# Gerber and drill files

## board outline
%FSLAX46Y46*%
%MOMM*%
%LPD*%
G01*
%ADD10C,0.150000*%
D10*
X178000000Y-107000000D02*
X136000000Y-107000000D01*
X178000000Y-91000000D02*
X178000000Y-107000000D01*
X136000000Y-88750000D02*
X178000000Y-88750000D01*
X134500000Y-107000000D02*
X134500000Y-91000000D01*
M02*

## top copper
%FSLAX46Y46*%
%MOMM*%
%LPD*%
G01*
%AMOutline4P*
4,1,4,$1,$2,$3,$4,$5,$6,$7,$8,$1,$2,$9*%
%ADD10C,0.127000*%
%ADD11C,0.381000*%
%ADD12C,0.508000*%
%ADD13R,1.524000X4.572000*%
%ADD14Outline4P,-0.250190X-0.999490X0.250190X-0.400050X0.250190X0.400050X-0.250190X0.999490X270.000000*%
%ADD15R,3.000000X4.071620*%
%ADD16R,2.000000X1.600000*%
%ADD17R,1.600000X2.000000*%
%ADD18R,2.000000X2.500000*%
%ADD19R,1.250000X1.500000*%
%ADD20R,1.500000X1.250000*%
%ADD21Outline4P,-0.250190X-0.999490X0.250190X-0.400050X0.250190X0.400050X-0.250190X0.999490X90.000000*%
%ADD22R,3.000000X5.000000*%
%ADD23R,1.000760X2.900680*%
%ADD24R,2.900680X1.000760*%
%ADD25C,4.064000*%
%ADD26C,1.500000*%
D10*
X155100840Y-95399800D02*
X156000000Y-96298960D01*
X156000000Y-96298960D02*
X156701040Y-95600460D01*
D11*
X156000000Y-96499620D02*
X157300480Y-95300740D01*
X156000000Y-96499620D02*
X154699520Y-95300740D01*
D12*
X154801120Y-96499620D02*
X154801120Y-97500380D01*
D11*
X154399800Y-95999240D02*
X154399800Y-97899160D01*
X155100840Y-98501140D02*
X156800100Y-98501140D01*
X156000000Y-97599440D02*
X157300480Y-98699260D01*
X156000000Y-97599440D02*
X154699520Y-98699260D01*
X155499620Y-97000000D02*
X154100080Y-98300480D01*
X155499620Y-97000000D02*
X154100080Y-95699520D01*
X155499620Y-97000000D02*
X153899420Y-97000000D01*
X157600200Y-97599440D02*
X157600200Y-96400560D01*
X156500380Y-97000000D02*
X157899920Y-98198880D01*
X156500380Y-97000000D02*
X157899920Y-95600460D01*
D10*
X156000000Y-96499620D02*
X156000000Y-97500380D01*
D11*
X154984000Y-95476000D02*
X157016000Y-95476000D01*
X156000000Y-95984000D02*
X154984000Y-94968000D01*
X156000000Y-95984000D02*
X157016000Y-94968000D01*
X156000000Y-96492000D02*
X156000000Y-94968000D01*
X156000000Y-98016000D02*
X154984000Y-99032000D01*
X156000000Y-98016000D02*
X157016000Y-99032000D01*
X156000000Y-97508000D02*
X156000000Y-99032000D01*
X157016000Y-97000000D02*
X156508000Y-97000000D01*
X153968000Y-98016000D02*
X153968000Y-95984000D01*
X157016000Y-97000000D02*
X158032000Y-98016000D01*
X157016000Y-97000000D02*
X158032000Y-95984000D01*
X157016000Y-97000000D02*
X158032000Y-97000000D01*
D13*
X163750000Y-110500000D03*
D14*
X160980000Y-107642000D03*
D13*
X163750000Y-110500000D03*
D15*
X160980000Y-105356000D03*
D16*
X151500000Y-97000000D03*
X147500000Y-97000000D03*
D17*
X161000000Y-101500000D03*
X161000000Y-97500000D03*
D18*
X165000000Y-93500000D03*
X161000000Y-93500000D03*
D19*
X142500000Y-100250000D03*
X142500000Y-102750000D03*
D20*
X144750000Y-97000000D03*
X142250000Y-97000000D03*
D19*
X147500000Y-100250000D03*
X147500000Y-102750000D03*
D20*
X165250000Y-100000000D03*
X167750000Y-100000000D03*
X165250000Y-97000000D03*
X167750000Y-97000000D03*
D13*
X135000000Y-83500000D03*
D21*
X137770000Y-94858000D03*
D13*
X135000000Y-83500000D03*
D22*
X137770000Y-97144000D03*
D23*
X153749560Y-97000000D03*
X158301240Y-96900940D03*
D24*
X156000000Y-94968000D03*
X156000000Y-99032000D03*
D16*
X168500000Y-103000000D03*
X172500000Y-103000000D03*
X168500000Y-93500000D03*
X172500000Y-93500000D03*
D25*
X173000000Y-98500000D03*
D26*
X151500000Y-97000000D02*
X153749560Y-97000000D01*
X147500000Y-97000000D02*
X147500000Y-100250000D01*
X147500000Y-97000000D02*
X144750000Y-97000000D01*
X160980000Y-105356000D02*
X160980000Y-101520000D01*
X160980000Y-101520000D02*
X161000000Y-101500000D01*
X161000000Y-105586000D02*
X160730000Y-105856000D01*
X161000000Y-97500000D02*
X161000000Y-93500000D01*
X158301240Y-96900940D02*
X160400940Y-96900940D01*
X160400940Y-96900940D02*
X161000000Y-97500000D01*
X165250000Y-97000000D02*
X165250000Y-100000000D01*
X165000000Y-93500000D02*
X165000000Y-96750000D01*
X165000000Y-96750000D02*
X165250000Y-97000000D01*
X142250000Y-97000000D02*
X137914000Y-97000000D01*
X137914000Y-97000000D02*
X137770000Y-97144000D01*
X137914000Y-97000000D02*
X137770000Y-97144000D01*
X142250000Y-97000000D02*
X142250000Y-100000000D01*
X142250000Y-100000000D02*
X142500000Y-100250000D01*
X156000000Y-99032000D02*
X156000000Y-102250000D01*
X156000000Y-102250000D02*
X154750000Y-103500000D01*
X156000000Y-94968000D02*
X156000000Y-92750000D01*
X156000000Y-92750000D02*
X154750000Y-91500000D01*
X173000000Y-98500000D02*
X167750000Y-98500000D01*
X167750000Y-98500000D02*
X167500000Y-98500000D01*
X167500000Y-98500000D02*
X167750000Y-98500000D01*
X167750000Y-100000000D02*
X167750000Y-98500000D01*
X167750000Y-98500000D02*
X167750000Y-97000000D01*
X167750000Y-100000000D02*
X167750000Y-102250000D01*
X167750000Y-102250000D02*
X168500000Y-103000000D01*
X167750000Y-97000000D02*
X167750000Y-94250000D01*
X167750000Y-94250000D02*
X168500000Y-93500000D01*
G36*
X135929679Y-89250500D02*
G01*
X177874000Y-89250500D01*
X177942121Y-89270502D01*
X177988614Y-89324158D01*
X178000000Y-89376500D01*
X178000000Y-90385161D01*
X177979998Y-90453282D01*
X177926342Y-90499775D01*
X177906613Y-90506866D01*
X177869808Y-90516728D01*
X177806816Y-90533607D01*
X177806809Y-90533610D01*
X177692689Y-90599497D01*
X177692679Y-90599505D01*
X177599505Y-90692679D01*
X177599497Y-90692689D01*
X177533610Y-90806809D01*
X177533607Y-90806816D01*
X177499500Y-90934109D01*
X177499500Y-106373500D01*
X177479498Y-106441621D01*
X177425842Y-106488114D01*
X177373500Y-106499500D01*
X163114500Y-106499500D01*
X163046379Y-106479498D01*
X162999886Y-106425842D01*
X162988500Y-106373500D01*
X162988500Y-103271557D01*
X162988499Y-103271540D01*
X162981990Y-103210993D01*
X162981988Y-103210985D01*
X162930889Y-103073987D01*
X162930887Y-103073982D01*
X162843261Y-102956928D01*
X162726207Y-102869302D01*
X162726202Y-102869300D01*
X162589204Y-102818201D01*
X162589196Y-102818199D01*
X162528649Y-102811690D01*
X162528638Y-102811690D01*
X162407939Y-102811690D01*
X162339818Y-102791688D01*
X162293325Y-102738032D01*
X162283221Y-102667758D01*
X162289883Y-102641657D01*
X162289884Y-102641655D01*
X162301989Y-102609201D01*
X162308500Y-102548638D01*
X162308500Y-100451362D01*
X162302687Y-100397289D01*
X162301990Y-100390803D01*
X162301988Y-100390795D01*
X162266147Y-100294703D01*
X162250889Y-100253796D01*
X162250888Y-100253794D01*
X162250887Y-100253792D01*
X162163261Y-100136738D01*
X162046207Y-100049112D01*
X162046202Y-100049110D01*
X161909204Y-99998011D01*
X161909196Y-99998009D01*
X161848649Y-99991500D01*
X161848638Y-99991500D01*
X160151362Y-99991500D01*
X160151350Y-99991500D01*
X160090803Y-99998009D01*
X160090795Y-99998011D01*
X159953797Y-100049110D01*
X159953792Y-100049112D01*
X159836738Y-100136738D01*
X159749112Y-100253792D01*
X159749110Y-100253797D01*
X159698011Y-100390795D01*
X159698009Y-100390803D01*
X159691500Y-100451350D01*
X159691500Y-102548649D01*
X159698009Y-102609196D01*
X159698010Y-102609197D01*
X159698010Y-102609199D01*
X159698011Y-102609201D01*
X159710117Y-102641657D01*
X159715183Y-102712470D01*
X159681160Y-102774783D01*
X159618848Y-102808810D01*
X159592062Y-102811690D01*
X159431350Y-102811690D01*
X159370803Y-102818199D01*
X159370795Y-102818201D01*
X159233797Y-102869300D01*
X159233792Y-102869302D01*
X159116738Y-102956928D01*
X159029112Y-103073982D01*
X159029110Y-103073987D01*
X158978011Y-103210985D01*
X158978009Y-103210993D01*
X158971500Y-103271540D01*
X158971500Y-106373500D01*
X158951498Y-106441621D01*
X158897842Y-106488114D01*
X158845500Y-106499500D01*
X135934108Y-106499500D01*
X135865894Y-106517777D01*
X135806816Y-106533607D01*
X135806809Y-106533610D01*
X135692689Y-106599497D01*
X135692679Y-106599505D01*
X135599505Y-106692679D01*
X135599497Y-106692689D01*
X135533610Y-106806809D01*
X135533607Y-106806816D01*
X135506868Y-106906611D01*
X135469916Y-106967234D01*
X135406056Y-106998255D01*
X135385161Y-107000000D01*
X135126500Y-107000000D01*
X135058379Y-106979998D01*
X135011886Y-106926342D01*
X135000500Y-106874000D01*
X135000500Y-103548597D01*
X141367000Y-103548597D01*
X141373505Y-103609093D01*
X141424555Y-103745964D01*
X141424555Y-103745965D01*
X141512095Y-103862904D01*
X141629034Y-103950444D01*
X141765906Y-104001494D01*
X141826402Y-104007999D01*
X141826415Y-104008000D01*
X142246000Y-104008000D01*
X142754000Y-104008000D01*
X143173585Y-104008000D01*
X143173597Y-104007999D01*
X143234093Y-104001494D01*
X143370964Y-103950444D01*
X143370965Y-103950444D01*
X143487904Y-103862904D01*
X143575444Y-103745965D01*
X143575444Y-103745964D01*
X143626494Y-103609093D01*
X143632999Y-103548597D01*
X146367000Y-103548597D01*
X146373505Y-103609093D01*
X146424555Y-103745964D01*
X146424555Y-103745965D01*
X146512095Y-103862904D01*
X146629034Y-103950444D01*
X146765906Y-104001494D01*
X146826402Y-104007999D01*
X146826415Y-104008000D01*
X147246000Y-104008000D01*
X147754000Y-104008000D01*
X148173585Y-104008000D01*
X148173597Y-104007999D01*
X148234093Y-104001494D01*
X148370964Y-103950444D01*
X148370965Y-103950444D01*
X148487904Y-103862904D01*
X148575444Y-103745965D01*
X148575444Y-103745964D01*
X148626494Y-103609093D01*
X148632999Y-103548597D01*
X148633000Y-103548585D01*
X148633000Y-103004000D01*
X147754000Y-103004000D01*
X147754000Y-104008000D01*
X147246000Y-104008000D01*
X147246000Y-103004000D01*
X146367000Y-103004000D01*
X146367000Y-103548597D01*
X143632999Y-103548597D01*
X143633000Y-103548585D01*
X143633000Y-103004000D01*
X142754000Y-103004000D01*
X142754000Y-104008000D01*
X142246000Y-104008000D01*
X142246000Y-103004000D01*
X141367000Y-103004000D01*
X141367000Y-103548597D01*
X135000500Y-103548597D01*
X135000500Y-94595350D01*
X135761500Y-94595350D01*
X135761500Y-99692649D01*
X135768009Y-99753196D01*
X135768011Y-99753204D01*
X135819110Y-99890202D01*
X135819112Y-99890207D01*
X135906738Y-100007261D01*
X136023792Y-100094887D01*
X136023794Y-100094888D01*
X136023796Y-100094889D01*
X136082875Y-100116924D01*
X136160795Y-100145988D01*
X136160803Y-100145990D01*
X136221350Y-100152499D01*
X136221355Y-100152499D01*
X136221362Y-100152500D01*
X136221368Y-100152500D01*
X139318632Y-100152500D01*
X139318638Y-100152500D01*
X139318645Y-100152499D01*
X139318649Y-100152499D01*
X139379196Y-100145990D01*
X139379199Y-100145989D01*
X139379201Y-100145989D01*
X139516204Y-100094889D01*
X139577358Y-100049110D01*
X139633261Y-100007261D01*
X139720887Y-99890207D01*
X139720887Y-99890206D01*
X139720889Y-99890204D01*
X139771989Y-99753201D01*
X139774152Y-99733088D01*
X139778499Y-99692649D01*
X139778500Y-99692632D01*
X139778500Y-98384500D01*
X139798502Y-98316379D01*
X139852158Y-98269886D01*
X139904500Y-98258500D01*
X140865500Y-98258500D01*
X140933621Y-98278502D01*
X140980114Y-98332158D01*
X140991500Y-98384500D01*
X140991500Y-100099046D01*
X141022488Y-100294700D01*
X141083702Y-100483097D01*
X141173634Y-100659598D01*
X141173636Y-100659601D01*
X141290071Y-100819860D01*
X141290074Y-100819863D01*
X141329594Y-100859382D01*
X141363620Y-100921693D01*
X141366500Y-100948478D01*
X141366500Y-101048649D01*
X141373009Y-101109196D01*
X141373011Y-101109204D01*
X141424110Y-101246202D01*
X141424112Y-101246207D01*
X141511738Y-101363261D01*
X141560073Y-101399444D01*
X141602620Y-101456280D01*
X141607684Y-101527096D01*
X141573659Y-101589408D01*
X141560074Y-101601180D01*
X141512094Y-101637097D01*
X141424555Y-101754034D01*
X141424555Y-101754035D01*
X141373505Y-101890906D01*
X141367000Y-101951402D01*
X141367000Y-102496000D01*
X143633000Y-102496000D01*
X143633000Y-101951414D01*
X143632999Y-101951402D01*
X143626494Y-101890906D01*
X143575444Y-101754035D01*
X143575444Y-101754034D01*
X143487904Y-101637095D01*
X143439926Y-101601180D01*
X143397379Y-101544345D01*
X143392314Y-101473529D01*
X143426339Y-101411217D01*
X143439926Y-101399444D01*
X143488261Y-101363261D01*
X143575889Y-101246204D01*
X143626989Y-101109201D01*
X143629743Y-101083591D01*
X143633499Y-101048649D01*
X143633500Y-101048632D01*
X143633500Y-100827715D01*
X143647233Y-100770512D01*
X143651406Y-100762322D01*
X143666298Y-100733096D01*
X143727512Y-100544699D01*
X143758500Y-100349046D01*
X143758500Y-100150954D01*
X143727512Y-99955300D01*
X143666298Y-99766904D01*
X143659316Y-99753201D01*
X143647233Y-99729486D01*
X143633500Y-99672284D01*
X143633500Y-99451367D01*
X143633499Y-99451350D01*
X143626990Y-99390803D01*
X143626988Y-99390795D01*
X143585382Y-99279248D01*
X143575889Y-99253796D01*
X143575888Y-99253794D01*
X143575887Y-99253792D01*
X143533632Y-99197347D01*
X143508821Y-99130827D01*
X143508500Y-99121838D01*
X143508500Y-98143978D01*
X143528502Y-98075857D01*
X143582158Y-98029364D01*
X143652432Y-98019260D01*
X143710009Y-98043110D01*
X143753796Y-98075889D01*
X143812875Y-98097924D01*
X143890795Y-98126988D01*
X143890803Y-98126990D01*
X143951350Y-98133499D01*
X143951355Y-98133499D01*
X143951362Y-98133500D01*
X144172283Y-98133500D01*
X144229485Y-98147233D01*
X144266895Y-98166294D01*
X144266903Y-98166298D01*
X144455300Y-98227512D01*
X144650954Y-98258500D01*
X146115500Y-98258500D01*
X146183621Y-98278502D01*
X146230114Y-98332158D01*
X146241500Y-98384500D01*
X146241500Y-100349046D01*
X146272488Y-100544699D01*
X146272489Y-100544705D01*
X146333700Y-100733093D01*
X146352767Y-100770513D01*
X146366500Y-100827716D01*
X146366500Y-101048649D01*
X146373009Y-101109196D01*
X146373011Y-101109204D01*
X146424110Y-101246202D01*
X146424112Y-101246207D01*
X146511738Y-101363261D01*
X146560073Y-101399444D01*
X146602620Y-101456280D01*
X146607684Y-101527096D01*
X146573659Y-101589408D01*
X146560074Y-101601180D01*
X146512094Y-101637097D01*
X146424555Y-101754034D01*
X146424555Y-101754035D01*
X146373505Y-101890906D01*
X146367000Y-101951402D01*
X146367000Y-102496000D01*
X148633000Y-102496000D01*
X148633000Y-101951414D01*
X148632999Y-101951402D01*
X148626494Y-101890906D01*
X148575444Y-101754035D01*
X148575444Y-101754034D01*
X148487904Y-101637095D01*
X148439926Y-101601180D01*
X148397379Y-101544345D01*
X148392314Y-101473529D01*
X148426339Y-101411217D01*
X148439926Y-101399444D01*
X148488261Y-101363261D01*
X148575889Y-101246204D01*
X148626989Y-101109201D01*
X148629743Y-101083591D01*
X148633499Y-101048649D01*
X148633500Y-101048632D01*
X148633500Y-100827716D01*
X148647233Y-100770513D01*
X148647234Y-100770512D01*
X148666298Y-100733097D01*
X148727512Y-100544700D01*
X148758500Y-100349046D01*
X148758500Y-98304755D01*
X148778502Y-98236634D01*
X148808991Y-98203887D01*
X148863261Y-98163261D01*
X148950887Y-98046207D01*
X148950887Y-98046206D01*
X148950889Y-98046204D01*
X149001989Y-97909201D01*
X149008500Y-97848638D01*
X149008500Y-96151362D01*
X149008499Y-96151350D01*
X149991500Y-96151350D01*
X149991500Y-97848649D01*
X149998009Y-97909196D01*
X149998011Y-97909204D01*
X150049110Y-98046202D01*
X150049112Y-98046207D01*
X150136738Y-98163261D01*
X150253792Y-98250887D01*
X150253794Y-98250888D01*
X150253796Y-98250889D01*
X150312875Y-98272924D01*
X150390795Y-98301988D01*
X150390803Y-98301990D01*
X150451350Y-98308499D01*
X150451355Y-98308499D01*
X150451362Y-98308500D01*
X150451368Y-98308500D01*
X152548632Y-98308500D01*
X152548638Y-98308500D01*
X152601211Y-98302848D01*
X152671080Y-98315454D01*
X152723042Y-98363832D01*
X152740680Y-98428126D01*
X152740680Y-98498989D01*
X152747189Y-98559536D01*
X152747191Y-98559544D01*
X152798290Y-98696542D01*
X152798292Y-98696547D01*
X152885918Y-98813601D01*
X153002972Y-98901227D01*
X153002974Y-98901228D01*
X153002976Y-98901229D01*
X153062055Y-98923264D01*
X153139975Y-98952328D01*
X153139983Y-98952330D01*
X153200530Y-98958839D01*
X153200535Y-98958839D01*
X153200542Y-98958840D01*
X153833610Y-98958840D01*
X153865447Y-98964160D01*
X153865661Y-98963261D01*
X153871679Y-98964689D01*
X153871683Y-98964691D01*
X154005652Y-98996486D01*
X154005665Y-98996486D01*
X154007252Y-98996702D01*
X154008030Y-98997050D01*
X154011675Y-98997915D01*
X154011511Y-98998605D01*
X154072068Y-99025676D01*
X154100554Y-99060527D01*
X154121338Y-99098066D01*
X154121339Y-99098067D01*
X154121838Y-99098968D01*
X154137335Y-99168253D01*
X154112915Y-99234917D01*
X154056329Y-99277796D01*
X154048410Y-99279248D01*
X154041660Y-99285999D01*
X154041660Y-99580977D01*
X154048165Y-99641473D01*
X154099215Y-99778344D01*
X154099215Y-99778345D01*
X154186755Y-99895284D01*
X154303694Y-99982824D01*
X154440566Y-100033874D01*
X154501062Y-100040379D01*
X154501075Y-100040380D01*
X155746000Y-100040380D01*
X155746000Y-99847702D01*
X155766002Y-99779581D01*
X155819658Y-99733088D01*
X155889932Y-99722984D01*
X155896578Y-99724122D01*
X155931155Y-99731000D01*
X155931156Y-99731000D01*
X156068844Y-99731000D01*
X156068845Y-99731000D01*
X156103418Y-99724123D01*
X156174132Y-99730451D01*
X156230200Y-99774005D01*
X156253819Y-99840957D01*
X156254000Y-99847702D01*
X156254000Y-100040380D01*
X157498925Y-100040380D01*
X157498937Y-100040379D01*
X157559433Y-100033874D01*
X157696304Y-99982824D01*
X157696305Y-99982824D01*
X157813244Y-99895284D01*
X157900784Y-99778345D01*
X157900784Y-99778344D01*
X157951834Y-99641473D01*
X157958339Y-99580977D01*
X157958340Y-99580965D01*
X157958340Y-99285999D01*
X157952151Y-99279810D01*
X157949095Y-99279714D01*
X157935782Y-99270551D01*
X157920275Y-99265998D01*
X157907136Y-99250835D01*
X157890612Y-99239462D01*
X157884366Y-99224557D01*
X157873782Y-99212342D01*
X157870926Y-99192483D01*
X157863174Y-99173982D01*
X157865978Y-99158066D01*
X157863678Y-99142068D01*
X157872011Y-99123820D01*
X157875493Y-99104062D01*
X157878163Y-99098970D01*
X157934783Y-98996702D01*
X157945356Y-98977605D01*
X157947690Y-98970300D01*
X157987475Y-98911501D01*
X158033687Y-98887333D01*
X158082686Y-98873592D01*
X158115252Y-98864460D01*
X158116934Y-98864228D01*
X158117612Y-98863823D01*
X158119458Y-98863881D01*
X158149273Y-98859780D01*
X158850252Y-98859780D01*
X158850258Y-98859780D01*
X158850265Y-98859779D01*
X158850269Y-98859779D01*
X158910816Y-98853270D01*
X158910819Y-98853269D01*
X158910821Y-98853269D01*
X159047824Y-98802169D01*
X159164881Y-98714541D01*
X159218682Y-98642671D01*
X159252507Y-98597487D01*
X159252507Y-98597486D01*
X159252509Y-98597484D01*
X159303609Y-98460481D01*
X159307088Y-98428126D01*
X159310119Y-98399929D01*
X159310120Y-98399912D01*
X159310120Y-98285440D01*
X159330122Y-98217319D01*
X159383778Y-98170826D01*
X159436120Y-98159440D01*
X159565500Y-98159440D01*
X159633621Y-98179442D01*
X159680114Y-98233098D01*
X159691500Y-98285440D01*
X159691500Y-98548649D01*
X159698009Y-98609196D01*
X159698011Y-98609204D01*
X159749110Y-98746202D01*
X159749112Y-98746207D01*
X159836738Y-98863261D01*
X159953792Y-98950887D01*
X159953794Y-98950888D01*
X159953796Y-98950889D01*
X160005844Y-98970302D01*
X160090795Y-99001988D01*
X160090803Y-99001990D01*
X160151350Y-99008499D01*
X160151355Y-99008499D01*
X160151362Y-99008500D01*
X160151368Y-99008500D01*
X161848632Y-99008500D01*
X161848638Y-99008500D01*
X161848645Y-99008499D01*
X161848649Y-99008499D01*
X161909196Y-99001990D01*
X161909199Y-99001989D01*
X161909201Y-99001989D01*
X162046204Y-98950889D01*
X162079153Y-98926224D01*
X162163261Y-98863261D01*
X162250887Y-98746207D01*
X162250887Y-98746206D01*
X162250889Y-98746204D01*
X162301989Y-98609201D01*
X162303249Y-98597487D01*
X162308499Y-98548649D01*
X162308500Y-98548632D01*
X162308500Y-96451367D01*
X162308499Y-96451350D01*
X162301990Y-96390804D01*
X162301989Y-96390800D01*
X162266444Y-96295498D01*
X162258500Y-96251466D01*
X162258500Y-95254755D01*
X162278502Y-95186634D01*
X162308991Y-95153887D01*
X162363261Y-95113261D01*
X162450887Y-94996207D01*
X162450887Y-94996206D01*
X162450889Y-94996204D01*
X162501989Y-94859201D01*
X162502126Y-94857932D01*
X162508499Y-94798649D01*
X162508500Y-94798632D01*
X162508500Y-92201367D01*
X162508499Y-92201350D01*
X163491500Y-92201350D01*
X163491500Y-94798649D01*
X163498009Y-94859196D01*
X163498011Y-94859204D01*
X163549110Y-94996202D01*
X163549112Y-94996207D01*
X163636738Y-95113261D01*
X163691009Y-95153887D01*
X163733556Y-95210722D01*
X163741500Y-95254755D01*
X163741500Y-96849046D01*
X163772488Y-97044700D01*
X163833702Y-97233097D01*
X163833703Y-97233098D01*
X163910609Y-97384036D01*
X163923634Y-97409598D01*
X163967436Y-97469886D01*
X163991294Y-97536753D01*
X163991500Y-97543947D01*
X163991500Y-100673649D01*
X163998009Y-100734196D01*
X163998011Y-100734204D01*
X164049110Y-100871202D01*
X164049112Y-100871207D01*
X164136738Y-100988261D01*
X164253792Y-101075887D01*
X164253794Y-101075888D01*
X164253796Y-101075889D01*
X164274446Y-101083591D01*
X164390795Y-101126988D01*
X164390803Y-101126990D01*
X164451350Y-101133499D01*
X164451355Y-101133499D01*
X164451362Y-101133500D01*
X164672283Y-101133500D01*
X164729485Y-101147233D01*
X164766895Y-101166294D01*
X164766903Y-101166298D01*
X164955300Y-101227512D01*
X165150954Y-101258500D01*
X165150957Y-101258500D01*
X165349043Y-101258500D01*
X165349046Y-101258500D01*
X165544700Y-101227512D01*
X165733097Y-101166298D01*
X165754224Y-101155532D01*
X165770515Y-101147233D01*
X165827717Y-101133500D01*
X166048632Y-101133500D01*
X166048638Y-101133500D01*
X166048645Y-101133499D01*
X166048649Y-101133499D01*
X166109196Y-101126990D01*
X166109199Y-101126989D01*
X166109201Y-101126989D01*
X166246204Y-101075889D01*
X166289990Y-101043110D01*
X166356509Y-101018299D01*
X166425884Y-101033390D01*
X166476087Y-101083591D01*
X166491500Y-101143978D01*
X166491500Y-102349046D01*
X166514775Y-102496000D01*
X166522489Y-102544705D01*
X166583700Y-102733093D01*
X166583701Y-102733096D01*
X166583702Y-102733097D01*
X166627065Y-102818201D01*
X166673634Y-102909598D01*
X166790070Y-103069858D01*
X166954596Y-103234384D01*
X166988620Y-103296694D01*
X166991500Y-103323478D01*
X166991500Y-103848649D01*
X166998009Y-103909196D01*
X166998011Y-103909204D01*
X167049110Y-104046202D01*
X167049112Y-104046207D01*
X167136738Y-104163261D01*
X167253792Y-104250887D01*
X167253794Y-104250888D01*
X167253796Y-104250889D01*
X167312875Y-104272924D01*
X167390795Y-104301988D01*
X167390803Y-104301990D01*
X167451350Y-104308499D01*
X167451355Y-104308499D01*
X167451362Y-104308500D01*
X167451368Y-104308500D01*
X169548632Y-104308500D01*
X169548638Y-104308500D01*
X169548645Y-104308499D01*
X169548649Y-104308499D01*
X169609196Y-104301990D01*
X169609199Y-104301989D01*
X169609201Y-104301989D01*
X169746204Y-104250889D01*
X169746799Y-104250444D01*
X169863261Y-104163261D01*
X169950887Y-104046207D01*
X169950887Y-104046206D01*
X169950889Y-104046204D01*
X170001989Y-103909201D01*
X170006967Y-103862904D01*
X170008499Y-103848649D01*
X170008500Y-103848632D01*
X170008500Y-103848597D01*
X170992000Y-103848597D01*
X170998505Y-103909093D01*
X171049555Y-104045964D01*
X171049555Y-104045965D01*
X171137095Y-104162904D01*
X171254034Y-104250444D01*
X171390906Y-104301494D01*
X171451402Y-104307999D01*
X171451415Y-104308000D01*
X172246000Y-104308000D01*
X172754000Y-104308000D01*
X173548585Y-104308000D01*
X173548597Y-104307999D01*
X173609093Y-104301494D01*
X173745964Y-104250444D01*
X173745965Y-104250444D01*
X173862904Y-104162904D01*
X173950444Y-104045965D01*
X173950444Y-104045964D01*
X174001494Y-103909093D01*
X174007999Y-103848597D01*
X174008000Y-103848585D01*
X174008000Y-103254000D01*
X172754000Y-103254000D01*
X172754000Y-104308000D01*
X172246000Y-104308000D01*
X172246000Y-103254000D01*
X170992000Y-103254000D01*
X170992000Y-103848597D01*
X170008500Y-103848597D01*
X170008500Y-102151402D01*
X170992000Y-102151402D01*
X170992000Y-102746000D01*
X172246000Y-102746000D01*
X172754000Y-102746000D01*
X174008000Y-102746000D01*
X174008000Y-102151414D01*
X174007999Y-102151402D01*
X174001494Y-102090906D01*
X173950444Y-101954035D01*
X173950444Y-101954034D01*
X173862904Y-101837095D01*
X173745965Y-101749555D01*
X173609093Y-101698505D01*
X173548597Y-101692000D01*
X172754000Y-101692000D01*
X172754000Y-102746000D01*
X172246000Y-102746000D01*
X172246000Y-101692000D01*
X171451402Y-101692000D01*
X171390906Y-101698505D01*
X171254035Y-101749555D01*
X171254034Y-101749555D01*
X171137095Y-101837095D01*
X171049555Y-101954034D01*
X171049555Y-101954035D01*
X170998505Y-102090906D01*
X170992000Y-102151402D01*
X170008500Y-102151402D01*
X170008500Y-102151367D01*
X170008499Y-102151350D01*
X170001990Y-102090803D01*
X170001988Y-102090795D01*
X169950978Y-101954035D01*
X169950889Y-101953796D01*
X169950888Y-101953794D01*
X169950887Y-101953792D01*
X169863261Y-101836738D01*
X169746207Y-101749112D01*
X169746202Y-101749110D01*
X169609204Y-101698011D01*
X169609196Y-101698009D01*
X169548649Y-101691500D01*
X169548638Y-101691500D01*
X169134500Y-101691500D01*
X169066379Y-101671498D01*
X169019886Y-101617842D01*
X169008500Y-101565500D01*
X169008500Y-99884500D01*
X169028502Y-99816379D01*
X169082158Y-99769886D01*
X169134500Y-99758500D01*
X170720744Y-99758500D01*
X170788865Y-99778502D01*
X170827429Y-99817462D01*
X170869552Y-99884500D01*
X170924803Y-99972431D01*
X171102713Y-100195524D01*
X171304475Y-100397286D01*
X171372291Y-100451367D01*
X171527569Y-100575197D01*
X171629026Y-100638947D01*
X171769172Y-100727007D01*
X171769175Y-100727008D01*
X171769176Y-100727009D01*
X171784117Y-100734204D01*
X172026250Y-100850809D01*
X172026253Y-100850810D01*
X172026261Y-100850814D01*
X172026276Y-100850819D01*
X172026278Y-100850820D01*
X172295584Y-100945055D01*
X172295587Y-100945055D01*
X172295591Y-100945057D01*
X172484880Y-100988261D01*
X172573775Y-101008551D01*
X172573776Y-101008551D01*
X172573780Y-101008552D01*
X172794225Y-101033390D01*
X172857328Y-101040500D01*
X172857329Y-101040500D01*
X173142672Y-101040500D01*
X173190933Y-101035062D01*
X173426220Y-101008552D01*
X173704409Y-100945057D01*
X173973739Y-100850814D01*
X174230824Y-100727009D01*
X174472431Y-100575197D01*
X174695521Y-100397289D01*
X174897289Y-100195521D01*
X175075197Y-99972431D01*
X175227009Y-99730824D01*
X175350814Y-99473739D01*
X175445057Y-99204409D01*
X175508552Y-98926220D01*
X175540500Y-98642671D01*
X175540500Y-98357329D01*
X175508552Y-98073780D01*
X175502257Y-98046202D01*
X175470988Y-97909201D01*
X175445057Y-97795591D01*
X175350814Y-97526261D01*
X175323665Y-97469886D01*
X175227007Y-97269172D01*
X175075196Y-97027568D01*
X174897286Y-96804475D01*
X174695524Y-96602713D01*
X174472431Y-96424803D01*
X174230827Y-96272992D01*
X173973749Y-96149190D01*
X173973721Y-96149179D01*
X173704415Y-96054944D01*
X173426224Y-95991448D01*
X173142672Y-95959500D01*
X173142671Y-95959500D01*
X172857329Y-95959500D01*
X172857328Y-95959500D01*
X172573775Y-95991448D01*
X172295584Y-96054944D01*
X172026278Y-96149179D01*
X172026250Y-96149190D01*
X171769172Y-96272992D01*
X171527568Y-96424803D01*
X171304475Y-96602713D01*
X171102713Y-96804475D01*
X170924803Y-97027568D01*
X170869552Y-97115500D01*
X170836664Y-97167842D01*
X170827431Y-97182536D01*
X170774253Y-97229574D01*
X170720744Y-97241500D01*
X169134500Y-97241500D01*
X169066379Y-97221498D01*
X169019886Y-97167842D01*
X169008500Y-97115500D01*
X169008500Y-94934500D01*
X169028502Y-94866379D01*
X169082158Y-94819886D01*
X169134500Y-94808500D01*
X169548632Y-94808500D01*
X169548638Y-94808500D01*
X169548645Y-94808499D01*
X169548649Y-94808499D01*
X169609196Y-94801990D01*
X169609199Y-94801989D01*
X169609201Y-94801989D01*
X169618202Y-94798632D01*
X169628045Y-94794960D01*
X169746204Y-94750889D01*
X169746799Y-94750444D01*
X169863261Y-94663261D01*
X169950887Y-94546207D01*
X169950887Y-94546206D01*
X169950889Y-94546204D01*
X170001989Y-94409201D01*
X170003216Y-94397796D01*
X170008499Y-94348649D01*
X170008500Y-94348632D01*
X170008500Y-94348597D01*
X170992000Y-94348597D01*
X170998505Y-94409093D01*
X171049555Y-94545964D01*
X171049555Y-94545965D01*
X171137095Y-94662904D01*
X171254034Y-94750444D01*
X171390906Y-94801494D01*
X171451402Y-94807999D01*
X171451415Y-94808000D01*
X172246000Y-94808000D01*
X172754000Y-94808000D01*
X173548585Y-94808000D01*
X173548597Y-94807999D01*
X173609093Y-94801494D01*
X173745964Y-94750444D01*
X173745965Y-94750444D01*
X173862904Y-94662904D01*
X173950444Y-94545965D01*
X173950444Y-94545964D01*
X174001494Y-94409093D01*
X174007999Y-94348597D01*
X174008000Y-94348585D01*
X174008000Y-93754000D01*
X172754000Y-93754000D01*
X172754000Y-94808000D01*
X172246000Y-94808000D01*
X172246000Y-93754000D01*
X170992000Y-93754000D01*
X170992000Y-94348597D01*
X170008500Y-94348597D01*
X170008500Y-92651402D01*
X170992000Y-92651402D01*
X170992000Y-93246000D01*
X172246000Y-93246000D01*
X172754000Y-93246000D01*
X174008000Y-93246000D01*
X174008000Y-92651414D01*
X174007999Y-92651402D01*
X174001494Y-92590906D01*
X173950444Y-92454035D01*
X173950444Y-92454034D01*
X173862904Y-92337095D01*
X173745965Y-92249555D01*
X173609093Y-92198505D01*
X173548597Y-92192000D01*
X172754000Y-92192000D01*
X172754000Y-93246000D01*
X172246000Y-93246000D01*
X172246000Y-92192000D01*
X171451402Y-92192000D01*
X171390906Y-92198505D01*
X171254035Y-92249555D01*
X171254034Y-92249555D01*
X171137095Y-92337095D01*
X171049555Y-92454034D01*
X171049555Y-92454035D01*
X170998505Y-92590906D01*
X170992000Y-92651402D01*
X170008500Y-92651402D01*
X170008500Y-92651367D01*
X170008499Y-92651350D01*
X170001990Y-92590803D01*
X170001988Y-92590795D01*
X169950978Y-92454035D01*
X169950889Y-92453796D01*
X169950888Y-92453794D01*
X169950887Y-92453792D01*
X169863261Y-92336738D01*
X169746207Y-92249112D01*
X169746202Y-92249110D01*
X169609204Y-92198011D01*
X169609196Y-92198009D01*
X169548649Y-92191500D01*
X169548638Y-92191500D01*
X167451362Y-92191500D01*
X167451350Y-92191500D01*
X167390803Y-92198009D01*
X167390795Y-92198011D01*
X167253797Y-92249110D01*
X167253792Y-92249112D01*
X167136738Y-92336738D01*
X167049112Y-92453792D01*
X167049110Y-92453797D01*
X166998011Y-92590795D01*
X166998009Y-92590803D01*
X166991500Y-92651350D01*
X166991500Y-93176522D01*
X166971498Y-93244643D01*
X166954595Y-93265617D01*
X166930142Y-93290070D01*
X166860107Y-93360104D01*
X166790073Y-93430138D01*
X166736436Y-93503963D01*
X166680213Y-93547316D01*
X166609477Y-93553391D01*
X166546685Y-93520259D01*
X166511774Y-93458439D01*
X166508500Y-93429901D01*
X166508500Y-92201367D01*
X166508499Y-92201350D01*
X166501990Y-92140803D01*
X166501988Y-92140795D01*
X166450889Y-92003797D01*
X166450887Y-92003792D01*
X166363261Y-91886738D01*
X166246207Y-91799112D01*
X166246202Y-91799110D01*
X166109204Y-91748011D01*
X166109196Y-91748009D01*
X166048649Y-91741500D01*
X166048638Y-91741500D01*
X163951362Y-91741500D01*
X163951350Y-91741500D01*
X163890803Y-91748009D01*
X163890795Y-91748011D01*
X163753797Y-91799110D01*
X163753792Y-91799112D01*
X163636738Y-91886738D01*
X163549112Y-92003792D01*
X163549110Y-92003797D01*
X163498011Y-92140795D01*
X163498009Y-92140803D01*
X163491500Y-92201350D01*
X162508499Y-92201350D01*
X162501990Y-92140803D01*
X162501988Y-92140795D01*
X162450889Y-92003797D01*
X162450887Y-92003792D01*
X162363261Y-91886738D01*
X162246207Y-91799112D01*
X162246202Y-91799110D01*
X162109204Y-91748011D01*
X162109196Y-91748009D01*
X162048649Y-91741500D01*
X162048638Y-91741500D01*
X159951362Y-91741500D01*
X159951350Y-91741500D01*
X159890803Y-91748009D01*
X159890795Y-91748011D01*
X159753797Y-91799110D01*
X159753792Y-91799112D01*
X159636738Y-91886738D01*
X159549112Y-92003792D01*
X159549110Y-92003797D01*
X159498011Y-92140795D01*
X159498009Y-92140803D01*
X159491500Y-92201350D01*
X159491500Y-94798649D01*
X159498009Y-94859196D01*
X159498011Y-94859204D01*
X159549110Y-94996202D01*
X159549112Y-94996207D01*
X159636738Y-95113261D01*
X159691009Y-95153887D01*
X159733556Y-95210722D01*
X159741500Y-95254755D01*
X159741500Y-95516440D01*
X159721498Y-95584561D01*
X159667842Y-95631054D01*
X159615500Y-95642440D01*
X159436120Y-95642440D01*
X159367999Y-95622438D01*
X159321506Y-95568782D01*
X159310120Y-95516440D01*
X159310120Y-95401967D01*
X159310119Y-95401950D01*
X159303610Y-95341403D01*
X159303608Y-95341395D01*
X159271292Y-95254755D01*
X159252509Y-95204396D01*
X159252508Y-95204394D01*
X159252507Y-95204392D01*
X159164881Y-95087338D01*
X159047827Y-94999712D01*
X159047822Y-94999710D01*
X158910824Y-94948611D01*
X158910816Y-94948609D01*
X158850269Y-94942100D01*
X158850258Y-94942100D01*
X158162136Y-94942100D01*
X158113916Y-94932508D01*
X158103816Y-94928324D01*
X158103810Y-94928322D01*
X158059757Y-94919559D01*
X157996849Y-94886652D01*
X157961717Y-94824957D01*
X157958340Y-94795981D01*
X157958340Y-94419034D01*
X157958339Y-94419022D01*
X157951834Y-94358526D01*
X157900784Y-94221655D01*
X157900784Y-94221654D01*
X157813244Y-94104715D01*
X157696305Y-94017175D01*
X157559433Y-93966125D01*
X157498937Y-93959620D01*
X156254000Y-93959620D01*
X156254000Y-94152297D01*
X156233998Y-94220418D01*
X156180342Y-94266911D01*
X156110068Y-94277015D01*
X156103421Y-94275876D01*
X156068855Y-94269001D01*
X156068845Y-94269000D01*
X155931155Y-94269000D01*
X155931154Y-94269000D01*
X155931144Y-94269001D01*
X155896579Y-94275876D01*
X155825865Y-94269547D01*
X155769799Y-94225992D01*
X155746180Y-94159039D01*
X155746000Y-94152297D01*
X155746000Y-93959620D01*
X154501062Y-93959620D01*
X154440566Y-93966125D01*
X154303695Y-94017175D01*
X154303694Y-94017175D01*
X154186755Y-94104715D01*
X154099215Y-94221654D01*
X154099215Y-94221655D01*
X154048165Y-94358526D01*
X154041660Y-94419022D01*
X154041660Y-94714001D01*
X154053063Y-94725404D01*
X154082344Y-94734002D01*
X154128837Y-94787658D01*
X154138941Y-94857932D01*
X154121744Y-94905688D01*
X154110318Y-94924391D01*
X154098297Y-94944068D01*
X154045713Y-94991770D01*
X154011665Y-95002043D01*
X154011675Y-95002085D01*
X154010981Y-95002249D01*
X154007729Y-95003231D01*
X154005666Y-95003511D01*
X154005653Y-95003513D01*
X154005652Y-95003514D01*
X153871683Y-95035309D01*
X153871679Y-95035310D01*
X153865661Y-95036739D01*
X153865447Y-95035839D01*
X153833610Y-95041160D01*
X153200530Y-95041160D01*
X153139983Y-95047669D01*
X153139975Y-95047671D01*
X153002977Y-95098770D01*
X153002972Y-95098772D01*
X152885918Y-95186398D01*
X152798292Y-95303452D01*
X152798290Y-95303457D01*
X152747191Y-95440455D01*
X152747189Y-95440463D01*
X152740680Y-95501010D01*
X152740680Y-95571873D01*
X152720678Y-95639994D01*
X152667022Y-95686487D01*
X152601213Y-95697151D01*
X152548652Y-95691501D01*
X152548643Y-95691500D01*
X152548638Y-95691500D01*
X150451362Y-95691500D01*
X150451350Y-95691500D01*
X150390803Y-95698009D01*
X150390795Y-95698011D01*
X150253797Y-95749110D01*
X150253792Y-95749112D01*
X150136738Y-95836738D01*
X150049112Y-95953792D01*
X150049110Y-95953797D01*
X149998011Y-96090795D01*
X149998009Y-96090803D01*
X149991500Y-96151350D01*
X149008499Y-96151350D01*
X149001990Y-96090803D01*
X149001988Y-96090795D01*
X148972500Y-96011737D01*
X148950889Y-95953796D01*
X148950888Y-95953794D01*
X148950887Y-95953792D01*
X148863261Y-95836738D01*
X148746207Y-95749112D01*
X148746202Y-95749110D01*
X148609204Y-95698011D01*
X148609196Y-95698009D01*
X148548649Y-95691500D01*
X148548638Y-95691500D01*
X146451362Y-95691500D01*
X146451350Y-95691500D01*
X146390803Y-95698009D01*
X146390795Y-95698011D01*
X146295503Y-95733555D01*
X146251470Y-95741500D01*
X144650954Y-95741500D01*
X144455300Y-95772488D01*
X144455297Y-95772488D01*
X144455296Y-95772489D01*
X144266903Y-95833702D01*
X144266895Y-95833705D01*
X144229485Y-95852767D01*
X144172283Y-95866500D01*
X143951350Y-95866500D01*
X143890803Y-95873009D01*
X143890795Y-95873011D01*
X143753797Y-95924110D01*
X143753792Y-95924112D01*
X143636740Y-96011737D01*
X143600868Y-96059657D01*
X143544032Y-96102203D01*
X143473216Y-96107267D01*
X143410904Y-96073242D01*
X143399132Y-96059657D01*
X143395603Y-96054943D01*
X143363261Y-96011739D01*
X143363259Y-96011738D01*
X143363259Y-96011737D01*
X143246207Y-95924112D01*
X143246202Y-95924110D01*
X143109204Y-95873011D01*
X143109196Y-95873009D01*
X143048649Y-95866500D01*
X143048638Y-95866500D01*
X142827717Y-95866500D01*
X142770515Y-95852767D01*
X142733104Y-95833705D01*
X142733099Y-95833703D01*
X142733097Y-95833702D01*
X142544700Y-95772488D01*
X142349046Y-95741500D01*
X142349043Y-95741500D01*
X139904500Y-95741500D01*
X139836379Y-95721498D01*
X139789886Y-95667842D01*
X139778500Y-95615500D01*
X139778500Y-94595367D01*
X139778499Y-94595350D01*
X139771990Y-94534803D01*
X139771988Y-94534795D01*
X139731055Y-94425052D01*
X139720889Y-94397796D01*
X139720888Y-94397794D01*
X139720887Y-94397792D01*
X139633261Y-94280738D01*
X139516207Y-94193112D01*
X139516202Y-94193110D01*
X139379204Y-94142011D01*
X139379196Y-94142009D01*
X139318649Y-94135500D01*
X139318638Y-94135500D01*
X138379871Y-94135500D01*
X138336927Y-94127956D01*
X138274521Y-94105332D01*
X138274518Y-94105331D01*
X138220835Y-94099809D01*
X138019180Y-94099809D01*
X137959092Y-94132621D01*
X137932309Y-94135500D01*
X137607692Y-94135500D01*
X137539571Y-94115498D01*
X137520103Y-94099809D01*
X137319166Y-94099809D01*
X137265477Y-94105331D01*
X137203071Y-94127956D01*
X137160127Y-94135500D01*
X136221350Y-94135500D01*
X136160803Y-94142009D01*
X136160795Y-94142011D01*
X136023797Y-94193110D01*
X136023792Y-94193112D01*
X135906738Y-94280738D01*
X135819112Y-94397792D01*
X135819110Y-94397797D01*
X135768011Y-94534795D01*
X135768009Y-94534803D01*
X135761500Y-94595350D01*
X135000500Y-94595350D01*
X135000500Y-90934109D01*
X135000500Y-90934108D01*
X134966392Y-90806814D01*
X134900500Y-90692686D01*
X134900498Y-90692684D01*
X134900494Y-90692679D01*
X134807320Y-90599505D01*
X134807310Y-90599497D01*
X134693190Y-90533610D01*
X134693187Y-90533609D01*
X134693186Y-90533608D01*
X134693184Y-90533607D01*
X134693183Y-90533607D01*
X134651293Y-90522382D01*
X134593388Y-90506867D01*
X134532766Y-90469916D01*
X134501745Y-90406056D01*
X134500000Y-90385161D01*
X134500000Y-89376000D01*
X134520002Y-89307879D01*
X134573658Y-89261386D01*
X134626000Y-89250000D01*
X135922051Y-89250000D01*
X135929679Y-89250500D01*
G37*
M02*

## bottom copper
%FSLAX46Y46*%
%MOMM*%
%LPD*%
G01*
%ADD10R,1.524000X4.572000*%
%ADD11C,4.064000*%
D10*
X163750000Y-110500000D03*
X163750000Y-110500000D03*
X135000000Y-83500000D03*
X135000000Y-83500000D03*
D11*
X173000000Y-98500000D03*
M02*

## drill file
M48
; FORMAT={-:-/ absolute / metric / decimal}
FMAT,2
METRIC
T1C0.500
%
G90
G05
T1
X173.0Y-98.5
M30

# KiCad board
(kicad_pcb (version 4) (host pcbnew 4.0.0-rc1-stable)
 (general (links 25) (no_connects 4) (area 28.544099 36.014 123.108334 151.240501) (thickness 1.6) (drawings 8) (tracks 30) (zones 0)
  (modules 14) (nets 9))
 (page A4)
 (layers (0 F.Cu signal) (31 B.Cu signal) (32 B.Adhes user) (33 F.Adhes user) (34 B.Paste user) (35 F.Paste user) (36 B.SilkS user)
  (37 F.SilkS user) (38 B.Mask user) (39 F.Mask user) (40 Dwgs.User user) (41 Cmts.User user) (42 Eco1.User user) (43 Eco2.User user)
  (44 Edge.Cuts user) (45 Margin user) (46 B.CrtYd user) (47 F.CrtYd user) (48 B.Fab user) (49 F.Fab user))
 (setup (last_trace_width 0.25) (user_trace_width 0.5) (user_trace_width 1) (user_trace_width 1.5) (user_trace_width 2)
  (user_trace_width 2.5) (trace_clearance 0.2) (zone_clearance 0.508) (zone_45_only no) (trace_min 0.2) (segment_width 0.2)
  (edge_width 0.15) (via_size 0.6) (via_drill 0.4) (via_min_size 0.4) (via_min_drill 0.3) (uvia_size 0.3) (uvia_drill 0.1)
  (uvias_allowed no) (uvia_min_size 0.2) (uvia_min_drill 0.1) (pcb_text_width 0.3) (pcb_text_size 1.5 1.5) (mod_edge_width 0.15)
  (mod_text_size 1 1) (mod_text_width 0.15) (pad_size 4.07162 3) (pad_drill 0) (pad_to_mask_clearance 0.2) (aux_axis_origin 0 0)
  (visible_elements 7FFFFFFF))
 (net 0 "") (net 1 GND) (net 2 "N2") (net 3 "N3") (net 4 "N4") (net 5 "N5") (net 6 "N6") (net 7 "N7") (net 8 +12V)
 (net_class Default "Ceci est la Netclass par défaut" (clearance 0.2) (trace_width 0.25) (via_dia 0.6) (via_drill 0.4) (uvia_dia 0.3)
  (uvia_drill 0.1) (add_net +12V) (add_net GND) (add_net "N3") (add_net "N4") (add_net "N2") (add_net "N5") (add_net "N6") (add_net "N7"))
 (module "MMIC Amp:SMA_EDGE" (layer F.Cu) (at 162.25 114.5 270)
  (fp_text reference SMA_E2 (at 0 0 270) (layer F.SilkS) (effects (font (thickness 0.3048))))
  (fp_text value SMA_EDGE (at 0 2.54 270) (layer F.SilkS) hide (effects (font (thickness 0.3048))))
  (pad 1 connect rect (at -4 -1.5 270) (size 4.572 1.524) (layers *.Cu F.Mask) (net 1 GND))
  (pad 1 connect trapezoid (at -6.858 1.27 270) (size 0.50038 1.39954) (rect_delta 0.59944 0) (layers F.Cu F.Mask) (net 1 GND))
  (pad 2 connect rect (at -4 -1.5 270) (size 4.572 1.524) (layers *.Cu F.Mask) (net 1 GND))
  (pad 3 connect rect (at -9.144 1.27 270) (size 4.07162 3) (layers F.Cu F.Mask) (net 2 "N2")))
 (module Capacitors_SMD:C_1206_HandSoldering (layer F.Cu) (at 149.5 97 180)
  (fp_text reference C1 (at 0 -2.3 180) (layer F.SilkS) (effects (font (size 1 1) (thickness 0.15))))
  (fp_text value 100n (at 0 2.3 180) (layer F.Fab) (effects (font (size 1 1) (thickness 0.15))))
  (pad 1 smd rect (at -2 0 180) (size 2 1.6) (layers F.Cu F.Paste F.Mask) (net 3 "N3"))
  (pad 2 smd rect (at 2 0 180) (size 2 1.6) (layers F.Cu F.Paste F.Mask) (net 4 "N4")))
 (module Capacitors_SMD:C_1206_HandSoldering (layer F.Cu) (at 161 99.5 90)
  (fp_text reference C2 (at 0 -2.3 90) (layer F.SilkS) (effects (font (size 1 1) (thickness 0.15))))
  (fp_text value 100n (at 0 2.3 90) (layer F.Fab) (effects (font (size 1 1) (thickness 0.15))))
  (pad 1 smd rect (at -2 0 90) (size 2 1.6) (layers F.Cu F.Paste F.Mask) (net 2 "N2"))
  (pad 2 smd rect (at 2 0 90) (size 2 1.6) (layers F.Cu F.Paste F.Mask) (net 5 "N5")))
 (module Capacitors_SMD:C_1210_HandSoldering (layer F.Cu) (at 163 93.5 180)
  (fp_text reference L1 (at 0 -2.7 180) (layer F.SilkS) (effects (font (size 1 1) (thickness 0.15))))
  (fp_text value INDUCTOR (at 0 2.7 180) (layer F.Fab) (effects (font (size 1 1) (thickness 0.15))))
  (pad 1 smd rect (at -2 0 180) (size 2 2.5) (layers F.Cu F.Paste F.Mask) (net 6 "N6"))
  (pad 2 smd rect (at 2 0 180) (size 2 2.5) (layers F.Cu F.Paste F.Mask) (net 5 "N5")))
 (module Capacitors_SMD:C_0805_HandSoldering (layer F.Cu) (at 142.5 101.5 270)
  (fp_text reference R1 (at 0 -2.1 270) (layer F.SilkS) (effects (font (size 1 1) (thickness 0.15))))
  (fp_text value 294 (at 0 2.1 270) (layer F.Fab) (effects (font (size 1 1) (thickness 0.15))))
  (pad 1 smd rect (at -1.25 0 270) (size 1.5 1.25) (layers F.Cu F.Paste F.Mask) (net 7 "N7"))
  (pad 2 smd rect (at 1.25 0 270) (size 1.5 1.25) (layers F.Cu F.Paste F.Mask) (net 1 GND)))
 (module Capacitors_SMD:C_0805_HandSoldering (layer F.Cu) (at 143.5 97 180)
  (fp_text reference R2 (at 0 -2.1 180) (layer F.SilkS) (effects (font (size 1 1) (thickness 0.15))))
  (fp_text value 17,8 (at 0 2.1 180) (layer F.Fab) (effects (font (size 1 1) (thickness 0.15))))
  (pad 1 smd rect (at -1.25 0 180) (size 1.5 1.25) (layers F.Cu F.Paste F.Mask) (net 4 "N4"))
  (pad 2 smd rect (at 1.25 0 180) (size 1.5 1.25) (layers F.Cu F.Paste F.Mask) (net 7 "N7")))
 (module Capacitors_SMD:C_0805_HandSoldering (layer F.Cu) (at 147.5 101.5 270)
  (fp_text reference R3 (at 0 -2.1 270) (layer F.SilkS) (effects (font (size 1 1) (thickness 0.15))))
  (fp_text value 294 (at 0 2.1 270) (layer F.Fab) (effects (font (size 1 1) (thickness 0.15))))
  (pad 1 smd rect (at -1.25 0 270) (size 1.5 1.25) (layers F.Cu F.Paste F.Mask) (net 4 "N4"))
  (pad 2 smd rect (at 1.25 0 270) (size 1.5 1.25) (layers F.Cu F.Paste F.Mask) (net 1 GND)))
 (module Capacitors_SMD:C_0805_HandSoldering (layer F.Cu) (at 166.5 100)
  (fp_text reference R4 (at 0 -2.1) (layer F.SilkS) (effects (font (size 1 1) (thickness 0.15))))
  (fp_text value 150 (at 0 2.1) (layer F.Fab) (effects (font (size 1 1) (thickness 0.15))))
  (pad 1 smd rect (at -1.25 0) (size 1.5 1.25) (layers F.Cu F.Paste F.Mask) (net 6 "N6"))
  (pad 2 smd rect (at 1.25 0) (size 1.5 1.25) (layers F.Cu F.Paste F.Mask) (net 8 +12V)))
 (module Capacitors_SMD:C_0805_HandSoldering (layer F.Cu) (at 166.5 97)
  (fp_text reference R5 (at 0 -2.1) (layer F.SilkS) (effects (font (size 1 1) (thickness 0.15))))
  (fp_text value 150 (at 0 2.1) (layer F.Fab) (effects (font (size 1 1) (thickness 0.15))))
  (pad 1 smd rect (at -1.25 0) (size 1.5 1.25) (layers F.Cu F.Paste F.Mask) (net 6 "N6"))
  (pad 2 smd rect (at 1.25 0) (size 1.5 1.25) (layers F.Cu F.Paste F.Mask) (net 8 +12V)))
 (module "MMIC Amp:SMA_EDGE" (layer F.Cu) (at 136.5 88 90)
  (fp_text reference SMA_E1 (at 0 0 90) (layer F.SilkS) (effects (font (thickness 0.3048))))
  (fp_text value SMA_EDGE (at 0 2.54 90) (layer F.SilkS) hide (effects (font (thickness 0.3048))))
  (pad 1 connect rect (at 4.5 -1.5 90) (size 4.572 1.524) (layers *.Cu F.Mask) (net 1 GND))
  (pad 1 connect trapezoid (at -6.858 1.27 90) (size 0.50038 1.39954) (rect_delta 0.59944 0) (layers F.Cu F.Mask) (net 1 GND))
  (pad 2 connect rect (at 4.5 -1.5 90) (size 4.572 1.524) (layers *.Cu F.Mask) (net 1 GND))
  (pad 3 connect rect (at -9.144 1.27 90) (size 5 3) (layers F.Cu F.Mask) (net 7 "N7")))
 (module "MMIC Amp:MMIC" (layer F.Cu) (at 156 97)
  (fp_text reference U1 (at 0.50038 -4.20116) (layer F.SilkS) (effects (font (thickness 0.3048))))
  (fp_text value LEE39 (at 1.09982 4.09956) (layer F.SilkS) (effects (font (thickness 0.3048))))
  (fp_line (start -0.89916 -1.6002) (end 0 -0.70104) (layer F.Cu) (width 0.127))
  (fp_line (start 0 -0.70104) (end 0.70104 -1.39954) (layer F.Cu) (width 0.127))
  (fp_line (start 0 -0.50038) (end 1.30048 -1.69926) (layer F.Cu) (width 0.381))
  (fp_line (start 0 -0.50038) (end -1.30048 -1.69926) (layer F.Cu) (width 0.381))
  (fp_line (start -1.19888 -0.50038) (end -1.19888 0.50038) (layer F.Cu) (width 0.508))
  (fp_line (start -1.6002 -1.00076) (end -1.6002 0.89916) (layer F.Cu) (width 0.381))
  (fp_line (start -0.89916 1.50114) (end 0.8001 1.50114) (layer F.Cu) (width 0.381))
  (fp_line (start 0 0.59944) (end 1.30048 1.69926) (layer F.Cu) (width 0.381))
  (fp_line (start 0 0.59944) (end -1.30048 1.69926) (layer F.Cu) (width 0.381))
  (fp_line (start -0.50038 0) (end -1.89992 1.30048) (layer F.Cu) (width 0.381))
  (fp_line (start -0.50038 0) (end -1.89992 -1.30048) (layer F.Cu) (width 0.381))
  (fp_line (start -0.50038 0) (end -2.10058 0) (layer F.Cu) (width 0.381))
  (fp_line (start 1.6002 0.59944) (end 1.6002 -0.59944) (layer F.Cu) (width 0.381))
  (fp_line (start 0.50038 0) (end 1.89992 1.19888) (layer F.Cu) (width 0.381))
  (fp_line (start 0.50038 0) (end 1.89992 -1.39954) (layer F.Cu) (width 0.381))
  (fp_line (start 0 -0.50038) (end 0 0.50038) (layer F.Cu) (width 0.127))
  (fp_line (start -1.016 -1.524) (end 1.016 -1.524) (layer F.Cu) (width 0.381))
  (fp_line (start 0 -1.016) (end -1.016 -2.032) (layer F.Cu) (width 0.381))
  (fp_line (start 0 -1.016) (end 1.016 -2.032) (layer F.Cu) (width 0.381))
  (fp_line (start 0 -0.508) (end 0 -2.032) (layer F.Cu) (width 0.381))
  (fp_line (start 0 1.016) (end -1.016 2.032) (layer F.Cu) (width 0.381))
  (fp_line (start 0 1.016) (end 1.016 2.032) (layer F.Cu) (width 0.381))
  (fp_line (start 0 0.508) (end 0 2.032) (layer F.Cu) (width 0.381))
  (fp_line (start 1.016 0) (end 0.508 0) (layer F.Cu) (width 0.381))
  (fp_line (start -2.032 1.016) (end -2.032 -1.016) (layer F.Cu) (width 0.381))
  (fp_line (start 1.016 0) (end 2.032 1.016) (layer F.Cu) (width 0.381))
  (fp_line (start 1.016 0) (end 2.032 -1.016) (layer F.Cu) (width 0.381))
  (fp_line (start 1.016 0) (end 2.032 0) (layer F.Cu) (width 0.381))
  (pad 1 smd rect (at -2.25044 0) (size 1.00076 2.90068) (layers F.Cu F.Paste F.Mask) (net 3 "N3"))
  (pad 3 smd rect (at 2.30124 -0.09906) (size 1.00076 2.90068) (layers F.Cu F.Paste F.Mask) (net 5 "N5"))
  (pad 4 smd rect (at 0 -2.032) (size 2.90068 1.00076) (layers F.Cu F.Paste F.Mask) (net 1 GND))
  (pad 2 smd rect (at 0 2.032) (size 2.90068 1.00076) (layers F.Cu F.Paste F.Mask) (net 1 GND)))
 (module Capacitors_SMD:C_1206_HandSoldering (layer F.Cu) (at 170.5 103)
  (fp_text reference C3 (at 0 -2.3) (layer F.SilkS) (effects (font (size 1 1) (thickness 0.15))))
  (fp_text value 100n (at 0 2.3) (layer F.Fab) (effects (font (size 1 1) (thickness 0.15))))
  (pad 1 smd rect (at -2 0) (size 2 1.6) (layers F.Cu F.Paste F.Mask) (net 8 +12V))
  (pad 2 smd rect (at 2 0) (size 2 1.6) (layers F.Cu F.Paste F.Mask) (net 1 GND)))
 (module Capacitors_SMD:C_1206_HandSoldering (layer F.Cu) (at 170.5 93.5)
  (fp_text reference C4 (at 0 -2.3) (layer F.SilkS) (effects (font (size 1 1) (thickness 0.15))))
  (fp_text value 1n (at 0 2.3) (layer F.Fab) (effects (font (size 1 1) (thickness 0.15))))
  (pad 1 smd rect (at -2 0) (size 2 1.6) (layers F.Cu F.Paste F.Mask) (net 8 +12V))
  (pad 2 smd rect (at 2 0) (size 2 1.6) (layers F.Cu F.Paste F.Mask) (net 1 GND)))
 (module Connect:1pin (layer F.Cu) (at 173 98.5)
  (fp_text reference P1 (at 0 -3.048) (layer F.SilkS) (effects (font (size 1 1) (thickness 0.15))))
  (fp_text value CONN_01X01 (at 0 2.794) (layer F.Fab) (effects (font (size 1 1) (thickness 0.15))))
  (pad 1 thru_hole circle (at 0 0) (size 4.064 4.064) (drill 0.5) (layers *.Cu *.Mask F.SilkS) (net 8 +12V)))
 (gr_line (start 178 107) (end 136 107) (angle 90) (layer Edge.Cuts) (width 0.15))
 (gr_line (start 178 91) (end 178 107) (angle 90) (layer Edge.Cuts) (width 0.15))
 (gr_line (start 136 88.75) (end 178 88.75) (angle 90) (layer Edge.Cuts) (width 0.15))
 (gr_line (start 134.5 107) (end 134.5 91) (angle 90) (layer Edge.Cuts) (width 0.15))
 (segment (start 151.5 97) (end 153.74956 97) (width 1.5) (layer F.Cu) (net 3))
 (segment (start 147.5 97) (end 147.5 100.25) (width 1.5) (layer F.Cu) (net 4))
 (segment (start 147.5 97) (end 144.75 97) (width 1.5) (layer F.Cu) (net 4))
 (segment (start 160.98 105.356) (end 160.98 101.52) (width 1.5) (layer F.Cu) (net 2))
 (segment (start 160.98 101.52) (end 161 101.5) (width 1.5) (layer F.Cu) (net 2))
 (segment (start 161 105.586) (end 160.73 105.856) (width 1.5) (layer F.Cu) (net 2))
 (segment (start 161 97.5) (end 161 93.5) (width 1.5) (layer F.Cu) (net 5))
 (segment (start 158.30124 96.90094) (end 160.40094 96.90094) (width 1.5) (layer F.Cu) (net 5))
 (segment (start 160.40094 96.90094) (end 161 97.5) (width 1.5) (layer F.Cu) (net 5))
 (segment (start 165.25 97) (end 165.25 100) (width 1.5) (layer F.Cu) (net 6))
 (segment (start 165 93.5) (end 165 96.75) (width 1.5) (layer F.Cu) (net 6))
 (segment (start 165 96.75) (end 165.25 97) (width 1.5) (layer F.Cu) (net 6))
 (segment (start 142.25 97) (end 137.914 97) (width 1.5) (layer F.Cu) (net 7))
 (segment (start 137.914 97) (end 137.77 97.144) (width 1.5) (layer F.Cu) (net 7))
 (segment (start 137.914 97) (end 137.77 97.144) (width 1.5) (layer F.Cu) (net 7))
 (segment (start 142.25 97) (end 142.25 100) (width 1.5) (layer F.Cu) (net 7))
 (segment (start 142.25 100) (end 142.5 100.25) (width 1.5) (layer F.Cu) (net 7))
 (segment (start 156 99.032) (end 156 102.25) (width 1.5) (layer F.Cu) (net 1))
 (segment (start 156 102.25) (end 154.75 103.5) (width 1.5) (layer F.Cu) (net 1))
 (segment (start 156 94.968) (end 156 92.75) (width 1.5) (layer F.Cu) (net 1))
 (segment (start 156 92.75) (end 154.75 91.5) (width 1.5) (layer F.Cu) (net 1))
 (segment (start 173 98.5) (end 167.75 98.5) (width 1.5) (layer F.Cu) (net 8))
 (segment (start 167.75 98.5) (end 167.5 98.5) (width 1.5) (layer F.Cu) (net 8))
 (segment (start 167.5 98.5) (end 167.75 98.5) (width 1.5) (layer F.Cu) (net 8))
 (segment (start 167.75 100) (end 167.75 98.5) (width 1.5) (layer F.Cu) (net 8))
 (segment (start 167.75 98.5) (end 167.75 97) (width 1.5) (layer F.Cu) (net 8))
 (segment (start 167.75 100) (end 167.75 102.25) (width 1.5) (layer F.Cu) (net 8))
 (segment (start 167.75 102.25) (end 168.5 103) (width 1.5) (layer F.Cu) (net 8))
 (segment (start 167.75 97) (end 167.75 94.25) (width 1.5) (layer F.Cu) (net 8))
 (segment (start 167.75 94.25) (end 168.5 93.5) (width 1.5) (layer F.Cu) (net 8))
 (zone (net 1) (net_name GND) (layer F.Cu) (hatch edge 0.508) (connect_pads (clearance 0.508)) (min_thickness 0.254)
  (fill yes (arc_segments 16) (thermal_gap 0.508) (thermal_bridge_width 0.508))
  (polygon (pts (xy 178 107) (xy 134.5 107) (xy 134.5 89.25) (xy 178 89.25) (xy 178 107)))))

